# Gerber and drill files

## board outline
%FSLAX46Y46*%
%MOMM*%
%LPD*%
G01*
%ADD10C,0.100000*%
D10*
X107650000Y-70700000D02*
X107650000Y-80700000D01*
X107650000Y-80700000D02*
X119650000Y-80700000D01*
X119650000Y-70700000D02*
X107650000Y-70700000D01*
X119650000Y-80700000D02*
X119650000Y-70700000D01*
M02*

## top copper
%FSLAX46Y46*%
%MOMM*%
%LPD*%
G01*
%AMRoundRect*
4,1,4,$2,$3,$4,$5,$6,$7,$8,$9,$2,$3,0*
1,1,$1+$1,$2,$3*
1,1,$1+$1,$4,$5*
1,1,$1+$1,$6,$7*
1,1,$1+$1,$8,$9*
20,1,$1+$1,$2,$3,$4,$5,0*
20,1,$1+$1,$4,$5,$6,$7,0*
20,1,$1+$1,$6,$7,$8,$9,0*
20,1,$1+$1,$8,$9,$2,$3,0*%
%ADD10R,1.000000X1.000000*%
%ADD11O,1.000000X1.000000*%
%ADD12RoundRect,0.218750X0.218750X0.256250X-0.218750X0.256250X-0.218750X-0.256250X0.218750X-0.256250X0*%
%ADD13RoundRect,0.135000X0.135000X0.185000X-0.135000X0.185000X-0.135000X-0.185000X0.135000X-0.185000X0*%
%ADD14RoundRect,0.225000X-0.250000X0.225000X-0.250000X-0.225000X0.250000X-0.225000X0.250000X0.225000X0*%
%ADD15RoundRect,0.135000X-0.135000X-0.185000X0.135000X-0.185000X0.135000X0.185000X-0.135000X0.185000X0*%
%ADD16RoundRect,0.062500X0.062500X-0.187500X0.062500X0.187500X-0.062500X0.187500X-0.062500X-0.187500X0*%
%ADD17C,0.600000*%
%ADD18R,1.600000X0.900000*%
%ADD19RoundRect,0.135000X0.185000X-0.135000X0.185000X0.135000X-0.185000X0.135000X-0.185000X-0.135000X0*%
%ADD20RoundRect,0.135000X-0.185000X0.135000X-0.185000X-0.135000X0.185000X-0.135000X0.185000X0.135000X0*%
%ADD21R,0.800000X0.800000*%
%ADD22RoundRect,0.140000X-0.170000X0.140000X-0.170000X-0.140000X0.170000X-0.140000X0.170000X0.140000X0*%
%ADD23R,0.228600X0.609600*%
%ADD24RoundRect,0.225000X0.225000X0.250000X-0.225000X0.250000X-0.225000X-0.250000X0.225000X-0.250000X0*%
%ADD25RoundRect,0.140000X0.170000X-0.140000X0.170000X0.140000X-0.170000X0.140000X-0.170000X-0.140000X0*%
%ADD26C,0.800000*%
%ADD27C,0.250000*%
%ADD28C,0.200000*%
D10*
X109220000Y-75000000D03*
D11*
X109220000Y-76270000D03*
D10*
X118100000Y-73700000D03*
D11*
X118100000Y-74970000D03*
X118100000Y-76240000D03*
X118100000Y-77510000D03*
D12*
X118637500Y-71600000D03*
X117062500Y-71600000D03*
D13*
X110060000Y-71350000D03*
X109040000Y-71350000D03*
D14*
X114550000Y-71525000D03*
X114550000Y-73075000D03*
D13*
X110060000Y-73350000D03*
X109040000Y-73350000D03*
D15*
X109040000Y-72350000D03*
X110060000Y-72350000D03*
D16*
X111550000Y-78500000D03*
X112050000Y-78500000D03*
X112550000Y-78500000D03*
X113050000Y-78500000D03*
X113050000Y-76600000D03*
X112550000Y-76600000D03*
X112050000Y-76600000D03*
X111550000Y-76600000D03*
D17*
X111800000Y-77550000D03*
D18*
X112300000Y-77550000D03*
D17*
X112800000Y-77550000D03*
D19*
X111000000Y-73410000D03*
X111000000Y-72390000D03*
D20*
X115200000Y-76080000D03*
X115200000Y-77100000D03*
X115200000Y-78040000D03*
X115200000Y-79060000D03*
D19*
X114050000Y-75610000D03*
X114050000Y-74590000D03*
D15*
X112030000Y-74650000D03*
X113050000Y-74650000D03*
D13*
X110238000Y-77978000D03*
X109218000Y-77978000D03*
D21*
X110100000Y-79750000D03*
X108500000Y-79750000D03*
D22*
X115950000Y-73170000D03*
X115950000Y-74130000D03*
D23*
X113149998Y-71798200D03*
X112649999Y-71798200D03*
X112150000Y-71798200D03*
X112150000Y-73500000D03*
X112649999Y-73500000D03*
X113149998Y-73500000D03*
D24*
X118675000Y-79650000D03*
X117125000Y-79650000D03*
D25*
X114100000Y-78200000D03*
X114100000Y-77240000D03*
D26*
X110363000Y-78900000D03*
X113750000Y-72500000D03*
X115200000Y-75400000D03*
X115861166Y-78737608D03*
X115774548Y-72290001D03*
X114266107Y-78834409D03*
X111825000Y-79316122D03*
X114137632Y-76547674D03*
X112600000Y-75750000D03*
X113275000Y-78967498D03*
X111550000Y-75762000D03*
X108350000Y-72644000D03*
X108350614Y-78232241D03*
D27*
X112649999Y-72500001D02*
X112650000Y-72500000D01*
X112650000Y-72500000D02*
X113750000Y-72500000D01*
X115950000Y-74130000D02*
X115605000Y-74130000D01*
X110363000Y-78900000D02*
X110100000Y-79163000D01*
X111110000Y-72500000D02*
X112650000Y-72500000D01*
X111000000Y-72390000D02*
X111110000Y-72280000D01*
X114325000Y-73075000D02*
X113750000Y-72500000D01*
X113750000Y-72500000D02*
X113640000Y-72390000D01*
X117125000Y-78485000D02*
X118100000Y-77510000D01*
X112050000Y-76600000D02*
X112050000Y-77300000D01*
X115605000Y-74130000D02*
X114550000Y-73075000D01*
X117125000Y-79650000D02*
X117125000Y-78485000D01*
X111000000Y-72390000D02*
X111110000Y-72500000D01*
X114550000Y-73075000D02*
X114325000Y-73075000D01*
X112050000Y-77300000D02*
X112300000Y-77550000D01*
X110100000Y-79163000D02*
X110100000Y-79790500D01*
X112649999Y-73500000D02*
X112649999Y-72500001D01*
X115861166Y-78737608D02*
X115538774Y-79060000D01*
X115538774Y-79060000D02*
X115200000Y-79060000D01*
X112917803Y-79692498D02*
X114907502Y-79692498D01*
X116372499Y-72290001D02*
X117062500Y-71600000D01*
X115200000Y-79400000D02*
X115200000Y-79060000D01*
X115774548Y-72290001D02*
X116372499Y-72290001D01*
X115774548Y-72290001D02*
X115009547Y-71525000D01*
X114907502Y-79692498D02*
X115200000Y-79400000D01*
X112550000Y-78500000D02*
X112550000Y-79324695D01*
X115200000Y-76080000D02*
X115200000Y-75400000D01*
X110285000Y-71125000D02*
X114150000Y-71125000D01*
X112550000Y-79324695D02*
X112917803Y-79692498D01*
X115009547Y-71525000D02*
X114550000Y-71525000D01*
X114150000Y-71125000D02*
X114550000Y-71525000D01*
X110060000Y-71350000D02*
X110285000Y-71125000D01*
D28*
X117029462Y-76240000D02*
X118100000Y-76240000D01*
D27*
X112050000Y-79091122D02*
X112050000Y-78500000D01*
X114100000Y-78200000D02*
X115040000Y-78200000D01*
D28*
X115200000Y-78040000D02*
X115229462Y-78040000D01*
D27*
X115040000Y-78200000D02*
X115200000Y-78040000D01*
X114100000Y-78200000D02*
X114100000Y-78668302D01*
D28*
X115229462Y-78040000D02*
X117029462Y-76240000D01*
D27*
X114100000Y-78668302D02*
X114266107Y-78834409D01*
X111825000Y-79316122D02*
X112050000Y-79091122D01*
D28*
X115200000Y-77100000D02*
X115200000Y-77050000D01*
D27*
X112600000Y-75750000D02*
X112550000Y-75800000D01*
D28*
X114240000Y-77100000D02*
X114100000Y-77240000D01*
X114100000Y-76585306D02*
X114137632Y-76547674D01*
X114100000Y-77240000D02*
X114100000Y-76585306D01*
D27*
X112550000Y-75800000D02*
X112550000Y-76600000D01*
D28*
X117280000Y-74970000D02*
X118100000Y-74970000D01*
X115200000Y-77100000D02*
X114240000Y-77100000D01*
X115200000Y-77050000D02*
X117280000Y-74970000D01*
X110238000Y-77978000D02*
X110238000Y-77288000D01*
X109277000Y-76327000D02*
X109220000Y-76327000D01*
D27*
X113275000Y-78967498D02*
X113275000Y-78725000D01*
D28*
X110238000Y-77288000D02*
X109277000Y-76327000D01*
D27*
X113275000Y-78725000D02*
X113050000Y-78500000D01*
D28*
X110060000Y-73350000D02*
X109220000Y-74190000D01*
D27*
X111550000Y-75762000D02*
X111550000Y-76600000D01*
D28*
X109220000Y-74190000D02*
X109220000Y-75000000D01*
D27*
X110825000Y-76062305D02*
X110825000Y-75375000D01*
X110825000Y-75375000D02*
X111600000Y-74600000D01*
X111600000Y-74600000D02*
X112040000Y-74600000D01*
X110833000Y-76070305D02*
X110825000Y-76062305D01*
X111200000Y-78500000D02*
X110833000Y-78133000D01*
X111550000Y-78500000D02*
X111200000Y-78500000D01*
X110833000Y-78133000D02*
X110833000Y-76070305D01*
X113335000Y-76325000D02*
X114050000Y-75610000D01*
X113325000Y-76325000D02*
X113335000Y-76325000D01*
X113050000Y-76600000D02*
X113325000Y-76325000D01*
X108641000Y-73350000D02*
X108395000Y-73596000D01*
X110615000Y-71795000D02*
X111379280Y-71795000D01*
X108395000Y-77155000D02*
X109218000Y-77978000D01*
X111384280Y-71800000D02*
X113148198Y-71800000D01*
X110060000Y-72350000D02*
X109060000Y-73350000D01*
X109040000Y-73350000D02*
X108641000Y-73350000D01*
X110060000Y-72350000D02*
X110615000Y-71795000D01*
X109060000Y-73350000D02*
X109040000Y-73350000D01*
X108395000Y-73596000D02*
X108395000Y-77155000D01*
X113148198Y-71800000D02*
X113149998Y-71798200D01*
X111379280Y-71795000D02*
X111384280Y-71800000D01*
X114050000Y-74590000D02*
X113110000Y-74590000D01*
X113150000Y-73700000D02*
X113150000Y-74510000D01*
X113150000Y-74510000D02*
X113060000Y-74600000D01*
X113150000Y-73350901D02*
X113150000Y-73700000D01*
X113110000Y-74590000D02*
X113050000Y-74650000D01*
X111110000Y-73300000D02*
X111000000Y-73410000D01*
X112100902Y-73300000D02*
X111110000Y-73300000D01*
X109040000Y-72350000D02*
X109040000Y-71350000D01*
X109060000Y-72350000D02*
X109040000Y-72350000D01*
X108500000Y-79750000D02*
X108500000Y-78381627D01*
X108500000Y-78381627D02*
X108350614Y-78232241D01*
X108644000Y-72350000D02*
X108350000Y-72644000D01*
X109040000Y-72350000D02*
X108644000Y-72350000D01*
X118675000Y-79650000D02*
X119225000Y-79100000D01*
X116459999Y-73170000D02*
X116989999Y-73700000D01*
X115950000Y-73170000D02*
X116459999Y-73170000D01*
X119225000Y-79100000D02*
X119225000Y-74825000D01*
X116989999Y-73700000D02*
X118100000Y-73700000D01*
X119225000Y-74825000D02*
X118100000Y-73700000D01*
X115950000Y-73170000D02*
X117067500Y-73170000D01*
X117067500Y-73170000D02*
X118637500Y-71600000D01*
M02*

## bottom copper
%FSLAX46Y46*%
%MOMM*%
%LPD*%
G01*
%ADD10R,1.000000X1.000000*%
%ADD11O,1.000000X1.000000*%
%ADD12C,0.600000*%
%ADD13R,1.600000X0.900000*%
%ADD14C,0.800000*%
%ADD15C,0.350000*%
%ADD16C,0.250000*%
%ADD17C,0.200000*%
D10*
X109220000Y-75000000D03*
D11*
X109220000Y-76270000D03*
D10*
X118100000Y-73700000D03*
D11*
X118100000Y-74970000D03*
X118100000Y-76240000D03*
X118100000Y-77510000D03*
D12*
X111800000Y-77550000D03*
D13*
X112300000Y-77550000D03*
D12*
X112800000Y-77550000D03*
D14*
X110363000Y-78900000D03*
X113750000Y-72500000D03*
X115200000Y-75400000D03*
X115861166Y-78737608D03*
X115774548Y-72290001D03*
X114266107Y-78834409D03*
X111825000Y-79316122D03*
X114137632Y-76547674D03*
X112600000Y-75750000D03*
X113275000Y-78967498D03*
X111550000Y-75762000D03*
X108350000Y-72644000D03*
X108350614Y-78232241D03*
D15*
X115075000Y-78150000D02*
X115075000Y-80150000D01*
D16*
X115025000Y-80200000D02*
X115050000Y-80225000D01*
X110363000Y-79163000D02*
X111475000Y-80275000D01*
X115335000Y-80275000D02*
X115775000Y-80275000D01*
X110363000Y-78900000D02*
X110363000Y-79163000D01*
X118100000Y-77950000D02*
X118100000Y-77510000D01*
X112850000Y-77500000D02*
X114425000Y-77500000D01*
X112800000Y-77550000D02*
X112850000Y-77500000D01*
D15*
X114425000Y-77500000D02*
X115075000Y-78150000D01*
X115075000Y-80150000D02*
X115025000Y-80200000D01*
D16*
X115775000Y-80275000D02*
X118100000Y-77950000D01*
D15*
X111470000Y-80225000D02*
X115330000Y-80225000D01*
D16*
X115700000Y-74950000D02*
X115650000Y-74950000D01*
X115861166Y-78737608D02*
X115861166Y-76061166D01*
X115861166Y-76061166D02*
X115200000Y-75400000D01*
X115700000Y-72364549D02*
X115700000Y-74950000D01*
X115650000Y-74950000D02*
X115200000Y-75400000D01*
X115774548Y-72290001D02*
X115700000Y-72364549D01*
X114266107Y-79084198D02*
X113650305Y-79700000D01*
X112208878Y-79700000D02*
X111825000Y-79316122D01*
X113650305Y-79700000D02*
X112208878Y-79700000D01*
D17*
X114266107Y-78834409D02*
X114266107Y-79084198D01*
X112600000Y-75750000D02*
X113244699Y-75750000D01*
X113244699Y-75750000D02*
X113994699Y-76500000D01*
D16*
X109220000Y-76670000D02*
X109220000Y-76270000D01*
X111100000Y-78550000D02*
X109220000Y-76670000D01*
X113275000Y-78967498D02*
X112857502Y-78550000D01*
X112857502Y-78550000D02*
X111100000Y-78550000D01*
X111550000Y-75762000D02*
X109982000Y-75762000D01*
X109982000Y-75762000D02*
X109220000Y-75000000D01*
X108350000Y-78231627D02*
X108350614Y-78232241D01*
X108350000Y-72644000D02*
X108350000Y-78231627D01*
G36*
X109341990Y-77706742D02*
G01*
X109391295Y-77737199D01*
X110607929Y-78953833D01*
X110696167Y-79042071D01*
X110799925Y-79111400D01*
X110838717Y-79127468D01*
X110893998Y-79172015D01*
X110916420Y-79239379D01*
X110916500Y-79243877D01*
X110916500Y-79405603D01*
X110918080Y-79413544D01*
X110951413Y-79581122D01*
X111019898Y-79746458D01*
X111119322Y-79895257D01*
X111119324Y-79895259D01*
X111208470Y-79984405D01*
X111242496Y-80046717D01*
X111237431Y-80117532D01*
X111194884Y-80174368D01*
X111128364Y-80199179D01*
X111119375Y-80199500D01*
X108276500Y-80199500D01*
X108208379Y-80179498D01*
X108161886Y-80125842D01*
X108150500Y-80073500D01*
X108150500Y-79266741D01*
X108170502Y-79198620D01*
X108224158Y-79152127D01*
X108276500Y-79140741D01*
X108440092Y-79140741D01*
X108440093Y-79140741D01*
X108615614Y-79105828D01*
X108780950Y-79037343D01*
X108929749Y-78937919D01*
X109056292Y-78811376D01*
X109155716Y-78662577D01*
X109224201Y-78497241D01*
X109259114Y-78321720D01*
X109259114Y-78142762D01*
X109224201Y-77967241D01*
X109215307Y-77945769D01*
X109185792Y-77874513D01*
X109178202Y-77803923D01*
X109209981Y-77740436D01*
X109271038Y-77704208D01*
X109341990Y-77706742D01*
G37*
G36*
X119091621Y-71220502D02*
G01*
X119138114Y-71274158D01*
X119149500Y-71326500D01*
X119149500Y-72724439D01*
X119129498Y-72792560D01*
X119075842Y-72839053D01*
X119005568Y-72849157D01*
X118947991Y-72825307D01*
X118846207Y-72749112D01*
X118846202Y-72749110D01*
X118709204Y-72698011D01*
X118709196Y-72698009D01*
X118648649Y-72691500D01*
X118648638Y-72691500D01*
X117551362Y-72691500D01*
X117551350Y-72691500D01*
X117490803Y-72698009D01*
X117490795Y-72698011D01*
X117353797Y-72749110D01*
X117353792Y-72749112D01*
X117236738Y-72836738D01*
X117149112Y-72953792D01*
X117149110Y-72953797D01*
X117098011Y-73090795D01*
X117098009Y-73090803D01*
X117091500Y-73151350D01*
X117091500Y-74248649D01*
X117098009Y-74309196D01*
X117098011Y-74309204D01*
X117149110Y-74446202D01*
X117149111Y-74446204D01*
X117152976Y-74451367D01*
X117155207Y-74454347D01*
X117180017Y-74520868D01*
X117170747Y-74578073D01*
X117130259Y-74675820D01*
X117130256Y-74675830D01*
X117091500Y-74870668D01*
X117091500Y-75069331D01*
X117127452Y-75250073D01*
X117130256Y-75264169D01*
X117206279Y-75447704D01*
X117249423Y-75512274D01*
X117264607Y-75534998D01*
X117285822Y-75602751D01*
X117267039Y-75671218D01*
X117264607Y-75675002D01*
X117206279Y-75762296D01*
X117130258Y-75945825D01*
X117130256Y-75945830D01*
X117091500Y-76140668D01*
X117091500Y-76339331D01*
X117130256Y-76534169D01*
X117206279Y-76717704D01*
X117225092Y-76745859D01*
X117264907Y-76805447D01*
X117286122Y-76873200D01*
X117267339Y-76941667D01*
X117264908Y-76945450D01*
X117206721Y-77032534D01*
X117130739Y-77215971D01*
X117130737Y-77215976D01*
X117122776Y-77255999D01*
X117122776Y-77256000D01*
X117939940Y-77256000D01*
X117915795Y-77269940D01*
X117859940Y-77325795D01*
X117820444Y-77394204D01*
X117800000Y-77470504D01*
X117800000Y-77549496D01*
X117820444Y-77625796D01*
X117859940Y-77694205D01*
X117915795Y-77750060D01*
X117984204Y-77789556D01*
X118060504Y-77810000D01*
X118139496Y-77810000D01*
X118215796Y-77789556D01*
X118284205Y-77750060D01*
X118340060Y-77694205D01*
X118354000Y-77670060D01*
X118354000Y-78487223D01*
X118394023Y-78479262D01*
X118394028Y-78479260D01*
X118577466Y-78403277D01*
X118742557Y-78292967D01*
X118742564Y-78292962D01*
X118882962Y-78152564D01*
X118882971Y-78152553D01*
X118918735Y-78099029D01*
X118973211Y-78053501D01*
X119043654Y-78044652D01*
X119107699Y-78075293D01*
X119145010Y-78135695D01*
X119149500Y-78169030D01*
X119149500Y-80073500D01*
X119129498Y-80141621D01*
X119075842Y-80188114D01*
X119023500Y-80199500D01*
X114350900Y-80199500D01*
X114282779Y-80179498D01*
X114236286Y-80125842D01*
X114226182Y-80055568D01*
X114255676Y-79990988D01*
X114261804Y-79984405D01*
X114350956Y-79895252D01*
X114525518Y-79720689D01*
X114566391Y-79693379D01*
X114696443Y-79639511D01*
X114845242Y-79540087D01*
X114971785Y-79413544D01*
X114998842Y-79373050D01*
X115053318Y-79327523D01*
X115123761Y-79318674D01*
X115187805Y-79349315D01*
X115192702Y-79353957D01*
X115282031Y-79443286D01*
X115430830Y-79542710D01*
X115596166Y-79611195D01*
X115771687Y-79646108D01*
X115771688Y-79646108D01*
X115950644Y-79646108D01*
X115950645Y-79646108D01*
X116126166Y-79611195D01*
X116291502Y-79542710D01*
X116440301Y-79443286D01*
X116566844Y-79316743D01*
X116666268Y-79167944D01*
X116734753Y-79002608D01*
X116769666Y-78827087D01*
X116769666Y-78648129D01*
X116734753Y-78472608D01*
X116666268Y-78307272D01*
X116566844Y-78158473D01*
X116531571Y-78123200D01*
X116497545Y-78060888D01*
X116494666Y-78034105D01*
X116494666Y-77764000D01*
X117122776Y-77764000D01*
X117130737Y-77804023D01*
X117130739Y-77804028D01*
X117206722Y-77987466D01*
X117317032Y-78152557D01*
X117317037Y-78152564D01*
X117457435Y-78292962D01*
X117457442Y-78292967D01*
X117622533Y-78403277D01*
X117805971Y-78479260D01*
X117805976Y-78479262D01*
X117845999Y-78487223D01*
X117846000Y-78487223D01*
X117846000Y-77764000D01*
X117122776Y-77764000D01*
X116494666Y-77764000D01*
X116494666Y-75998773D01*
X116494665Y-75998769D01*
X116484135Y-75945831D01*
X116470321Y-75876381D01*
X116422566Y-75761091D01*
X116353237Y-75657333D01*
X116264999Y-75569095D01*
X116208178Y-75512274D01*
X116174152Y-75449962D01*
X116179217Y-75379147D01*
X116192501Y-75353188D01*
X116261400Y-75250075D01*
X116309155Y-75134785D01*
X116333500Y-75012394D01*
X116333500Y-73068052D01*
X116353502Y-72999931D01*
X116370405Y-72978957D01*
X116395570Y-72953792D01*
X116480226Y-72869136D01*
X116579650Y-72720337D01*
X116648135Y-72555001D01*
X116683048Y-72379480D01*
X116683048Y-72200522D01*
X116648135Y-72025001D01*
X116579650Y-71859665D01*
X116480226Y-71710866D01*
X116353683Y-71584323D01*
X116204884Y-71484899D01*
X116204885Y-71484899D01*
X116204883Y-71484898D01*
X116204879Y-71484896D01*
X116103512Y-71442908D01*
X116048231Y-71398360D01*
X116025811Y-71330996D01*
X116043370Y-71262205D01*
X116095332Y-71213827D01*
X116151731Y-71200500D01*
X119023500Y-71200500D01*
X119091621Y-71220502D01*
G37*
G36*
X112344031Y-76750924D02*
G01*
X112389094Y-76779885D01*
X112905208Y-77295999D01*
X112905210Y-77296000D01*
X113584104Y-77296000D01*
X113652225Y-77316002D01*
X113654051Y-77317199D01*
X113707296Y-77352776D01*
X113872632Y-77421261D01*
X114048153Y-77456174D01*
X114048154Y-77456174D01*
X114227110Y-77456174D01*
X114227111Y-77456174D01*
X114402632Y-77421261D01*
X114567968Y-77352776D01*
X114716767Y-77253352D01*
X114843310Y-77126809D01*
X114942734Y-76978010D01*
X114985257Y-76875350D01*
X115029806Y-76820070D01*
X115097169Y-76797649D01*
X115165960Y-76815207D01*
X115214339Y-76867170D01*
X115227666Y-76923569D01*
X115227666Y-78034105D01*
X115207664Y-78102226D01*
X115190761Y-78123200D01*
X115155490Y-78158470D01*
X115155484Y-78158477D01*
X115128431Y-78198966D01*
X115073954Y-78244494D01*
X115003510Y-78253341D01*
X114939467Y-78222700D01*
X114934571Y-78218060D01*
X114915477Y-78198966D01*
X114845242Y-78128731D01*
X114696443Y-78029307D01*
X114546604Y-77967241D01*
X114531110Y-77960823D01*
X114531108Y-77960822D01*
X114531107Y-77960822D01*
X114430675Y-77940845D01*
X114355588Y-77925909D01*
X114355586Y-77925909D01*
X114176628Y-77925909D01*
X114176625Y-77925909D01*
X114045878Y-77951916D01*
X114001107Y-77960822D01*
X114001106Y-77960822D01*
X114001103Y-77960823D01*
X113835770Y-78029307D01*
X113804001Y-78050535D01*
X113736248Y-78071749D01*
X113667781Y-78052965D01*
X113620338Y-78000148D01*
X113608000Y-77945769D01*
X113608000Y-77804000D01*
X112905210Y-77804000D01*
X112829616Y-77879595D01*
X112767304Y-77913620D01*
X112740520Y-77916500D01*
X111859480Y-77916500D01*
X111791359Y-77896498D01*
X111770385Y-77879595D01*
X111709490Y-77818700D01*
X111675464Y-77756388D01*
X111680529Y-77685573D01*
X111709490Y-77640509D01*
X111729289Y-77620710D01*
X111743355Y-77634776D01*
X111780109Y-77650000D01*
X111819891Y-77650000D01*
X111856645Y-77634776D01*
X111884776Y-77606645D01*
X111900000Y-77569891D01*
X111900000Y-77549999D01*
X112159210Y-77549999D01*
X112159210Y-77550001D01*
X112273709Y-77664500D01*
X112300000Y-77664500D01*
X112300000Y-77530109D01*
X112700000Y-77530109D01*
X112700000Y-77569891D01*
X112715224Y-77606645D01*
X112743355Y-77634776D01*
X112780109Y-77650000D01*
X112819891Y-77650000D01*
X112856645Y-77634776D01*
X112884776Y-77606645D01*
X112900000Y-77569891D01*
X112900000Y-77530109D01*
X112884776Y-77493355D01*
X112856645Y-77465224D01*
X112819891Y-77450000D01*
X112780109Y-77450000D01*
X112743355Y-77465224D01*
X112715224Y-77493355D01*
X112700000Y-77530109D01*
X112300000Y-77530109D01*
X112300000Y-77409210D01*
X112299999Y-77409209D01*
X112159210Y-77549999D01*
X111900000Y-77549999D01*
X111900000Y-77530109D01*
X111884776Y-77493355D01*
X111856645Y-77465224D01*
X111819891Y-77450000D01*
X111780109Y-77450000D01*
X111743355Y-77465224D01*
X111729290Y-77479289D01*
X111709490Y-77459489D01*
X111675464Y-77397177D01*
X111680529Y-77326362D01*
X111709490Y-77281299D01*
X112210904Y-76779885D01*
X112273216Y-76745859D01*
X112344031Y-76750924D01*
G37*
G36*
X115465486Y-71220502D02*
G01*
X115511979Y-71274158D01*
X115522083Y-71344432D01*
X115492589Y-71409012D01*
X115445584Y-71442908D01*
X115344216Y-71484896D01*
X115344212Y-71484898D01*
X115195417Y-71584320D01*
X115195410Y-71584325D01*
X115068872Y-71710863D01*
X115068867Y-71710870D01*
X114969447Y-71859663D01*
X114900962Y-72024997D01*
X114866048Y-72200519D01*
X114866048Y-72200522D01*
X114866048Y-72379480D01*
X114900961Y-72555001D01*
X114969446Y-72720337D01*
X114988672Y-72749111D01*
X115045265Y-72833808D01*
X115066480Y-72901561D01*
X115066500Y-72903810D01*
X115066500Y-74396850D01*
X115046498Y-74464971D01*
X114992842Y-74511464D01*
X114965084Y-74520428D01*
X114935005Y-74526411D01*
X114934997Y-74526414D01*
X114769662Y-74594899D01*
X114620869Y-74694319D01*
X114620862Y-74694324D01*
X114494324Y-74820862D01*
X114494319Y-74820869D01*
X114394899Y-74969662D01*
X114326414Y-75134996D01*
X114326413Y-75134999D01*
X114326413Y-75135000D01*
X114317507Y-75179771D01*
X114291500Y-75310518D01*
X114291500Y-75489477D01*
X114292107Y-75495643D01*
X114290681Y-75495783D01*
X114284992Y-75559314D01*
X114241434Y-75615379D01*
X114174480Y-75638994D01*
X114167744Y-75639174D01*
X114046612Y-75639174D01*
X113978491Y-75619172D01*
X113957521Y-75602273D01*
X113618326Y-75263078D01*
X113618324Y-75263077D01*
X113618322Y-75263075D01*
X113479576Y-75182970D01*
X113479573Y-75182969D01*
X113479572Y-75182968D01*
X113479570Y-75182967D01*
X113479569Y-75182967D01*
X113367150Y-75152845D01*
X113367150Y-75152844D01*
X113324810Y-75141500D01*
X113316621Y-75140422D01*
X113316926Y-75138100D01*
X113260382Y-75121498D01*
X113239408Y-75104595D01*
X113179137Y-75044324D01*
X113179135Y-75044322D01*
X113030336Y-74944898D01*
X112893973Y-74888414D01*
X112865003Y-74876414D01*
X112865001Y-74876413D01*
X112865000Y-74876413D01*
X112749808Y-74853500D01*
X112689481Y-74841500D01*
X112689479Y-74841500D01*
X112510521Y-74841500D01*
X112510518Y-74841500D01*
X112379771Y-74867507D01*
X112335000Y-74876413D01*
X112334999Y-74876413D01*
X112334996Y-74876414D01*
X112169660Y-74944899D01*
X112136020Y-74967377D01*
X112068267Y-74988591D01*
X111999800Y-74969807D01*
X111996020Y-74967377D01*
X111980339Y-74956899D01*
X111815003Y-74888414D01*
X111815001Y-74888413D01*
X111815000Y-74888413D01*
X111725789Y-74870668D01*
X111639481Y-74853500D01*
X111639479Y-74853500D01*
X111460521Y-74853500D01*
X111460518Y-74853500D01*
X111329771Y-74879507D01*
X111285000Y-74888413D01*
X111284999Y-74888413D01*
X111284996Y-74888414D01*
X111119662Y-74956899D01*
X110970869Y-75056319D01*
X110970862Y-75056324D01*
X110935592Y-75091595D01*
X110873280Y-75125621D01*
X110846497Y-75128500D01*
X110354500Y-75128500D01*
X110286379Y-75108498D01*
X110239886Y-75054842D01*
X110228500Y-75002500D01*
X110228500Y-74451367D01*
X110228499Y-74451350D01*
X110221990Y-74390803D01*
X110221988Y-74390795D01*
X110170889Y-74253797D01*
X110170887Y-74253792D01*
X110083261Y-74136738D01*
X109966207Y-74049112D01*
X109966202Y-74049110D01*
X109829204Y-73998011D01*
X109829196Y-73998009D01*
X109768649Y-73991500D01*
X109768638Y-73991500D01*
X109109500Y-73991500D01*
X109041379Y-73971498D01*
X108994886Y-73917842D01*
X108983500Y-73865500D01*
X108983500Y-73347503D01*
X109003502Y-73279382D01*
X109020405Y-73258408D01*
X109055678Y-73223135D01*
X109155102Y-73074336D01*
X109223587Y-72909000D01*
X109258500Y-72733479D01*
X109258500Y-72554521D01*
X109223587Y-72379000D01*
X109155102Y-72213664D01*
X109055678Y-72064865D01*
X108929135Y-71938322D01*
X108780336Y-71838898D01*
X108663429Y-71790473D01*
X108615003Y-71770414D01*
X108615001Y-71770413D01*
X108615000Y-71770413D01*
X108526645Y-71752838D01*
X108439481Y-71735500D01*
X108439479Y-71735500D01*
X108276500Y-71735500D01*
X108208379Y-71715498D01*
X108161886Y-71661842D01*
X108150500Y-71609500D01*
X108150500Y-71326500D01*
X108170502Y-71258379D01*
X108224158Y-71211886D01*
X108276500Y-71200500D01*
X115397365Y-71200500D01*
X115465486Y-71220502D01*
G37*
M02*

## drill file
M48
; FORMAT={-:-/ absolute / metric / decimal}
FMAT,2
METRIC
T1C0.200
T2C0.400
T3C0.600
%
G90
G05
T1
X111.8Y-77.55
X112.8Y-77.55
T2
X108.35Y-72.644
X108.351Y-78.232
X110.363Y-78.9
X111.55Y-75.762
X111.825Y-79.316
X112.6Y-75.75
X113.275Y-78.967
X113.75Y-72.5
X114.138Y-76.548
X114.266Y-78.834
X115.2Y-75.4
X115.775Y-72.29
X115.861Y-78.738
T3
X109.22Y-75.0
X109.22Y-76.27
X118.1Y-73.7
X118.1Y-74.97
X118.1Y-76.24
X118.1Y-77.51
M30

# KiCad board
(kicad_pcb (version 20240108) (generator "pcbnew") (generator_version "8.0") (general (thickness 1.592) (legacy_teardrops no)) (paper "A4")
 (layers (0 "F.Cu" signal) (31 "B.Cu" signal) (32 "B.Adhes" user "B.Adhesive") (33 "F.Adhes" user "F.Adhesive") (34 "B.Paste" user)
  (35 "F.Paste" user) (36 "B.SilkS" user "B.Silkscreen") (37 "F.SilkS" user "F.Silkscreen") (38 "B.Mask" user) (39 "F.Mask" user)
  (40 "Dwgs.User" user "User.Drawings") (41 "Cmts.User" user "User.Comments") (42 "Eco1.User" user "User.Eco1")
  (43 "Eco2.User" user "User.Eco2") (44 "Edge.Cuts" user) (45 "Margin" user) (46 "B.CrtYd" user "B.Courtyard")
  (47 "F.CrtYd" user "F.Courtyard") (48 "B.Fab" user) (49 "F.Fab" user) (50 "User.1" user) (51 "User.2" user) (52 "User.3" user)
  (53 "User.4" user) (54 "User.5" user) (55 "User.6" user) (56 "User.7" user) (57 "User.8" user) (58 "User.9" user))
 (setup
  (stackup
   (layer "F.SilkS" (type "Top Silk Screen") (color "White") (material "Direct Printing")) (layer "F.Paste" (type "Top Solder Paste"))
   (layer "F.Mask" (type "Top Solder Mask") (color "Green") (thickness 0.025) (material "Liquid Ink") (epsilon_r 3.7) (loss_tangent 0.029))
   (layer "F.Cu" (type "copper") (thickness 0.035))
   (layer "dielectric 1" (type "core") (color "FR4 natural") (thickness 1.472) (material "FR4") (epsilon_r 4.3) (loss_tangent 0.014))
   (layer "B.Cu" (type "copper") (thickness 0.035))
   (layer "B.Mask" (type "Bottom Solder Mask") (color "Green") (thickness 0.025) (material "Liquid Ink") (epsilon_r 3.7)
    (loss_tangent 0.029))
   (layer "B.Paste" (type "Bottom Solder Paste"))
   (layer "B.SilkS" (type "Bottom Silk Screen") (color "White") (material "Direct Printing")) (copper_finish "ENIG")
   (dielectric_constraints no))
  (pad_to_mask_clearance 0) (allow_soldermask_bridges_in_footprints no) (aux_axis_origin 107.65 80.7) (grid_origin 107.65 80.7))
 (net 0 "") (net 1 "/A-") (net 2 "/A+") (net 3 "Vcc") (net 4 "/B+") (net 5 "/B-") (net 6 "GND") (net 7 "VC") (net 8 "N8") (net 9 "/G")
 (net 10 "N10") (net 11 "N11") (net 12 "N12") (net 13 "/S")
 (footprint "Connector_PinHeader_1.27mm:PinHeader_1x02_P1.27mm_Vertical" (layer "F.Cu") (at 109.22 75)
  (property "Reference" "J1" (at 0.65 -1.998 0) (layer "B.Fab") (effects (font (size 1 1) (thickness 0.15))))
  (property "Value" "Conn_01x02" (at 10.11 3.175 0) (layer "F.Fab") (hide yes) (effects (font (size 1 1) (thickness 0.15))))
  (pad "1" thru_hole rect (at 0 0) (size 1 1) (drill 0.6) (layers "*.Cu" "*.Mask") (remove_unused_layers no) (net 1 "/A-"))
  (pad "2" thru_hole oval (at 0 1.27) (size 1 1) (drill 0.6) (layers "*.Cu" "*.Mask") (remove_unused_layers no) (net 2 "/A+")))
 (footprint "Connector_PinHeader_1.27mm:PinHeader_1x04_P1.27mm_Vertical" (layer "F.Cu") (at 118.1 73.7)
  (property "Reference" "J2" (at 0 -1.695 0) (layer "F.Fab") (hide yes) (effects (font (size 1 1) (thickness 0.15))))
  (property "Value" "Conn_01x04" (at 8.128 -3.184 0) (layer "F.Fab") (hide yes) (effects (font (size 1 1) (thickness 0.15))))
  (pad "1" thru_hole rect (at 0 0) (size 1 1) (drill 0.6) (layers "*.Cu" "*.Mask") (remove_unused_layers no) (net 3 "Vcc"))
  (pad "2" thru_hole oval (at 0 1.27) (size 1 1) (drill 0.6) (layers "*.Cu" "*.Mask") (remove_unused_layers no) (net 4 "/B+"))
  (pad "3" thru_hole oval (at 0 2.54) (size 1 1) (drill 0.6) (layers "*.Cu" "*.Mask") (remove_unused_layers no) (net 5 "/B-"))
  (pad "4" thru_hole oval (at 0 3.81) (size 1 1) (drill 0.6) (layers "*.Cu" "*.Mask") (remove_unused_layers no) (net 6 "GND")))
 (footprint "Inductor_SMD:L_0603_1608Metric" (layer "F.Cu") (at 117.85 71.6 180)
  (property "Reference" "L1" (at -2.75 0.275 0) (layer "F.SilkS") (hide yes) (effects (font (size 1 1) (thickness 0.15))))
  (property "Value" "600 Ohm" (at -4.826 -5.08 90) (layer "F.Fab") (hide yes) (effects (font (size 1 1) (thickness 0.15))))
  (pad "1" smd roundrect (at -0.7875 0 180) (size 0.875 0.95) (layers "F.Cu" "F.Paste" "F.Mask") (roundrect_rratio 0.25) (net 3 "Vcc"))
  (pad "2" smd roundrect (at 0.7875 0 180) (size 0.875 0.95) (layers "F.Cu" "F.Paste" "F.Mask") (roundrect_rratio 0.25) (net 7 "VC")))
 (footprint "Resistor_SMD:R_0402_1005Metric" (layer "F.Cu") (at 109.55 71.35 180)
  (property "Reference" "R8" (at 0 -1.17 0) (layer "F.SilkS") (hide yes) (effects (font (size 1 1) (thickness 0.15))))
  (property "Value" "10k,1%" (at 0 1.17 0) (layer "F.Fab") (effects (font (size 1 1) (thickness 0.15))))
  (pad "1" smd roundrect (at -0.51 0 180) (size 0.54 0.64) (layers "F.Cu" "F.Paste" "F.Mask") (roundrect_rratio 0.25) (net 7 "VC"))
  (pad "2" smd roundrect (at 0.51 0 180) (size 0.54 0.64) (layers "F.Cu" "F.Paste" "F.Mask") (roundrect_rratio 0.25) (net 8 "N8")))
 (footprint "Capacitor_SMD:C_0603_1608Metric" (layer "F.Cu") (at 114.55 72.3 -90)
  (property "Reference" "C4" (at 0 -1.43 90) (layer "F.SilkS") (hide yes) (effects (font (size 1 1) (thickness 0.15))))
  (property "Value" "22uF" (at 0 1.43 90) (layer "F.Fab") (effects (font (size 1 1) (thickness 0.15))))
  (pad "1" smd roundrect (at -0.775 0 270) (size 0.9 0.95) (layers "F.Cu" "F.Paste" "F.Mask") (roundrect_rratio 0.25) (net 7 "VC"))
  (pad "2" smd roundrect (at 0.775 0 270) (size 0.9 0.95) (layers "F.Cu" "F.Paste" "F.Mask") (roundrect_rratio 0.25) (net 6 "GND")))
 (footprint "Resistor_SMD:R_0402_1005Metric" (layer "F.Cu") (at 109.55 73.35 180)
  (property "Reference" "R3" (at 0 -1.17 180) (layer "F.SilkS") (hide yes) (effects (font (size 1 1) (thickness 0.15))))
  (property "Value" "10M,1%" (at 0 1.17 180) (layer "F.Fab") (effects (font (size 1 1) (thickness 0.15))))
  (pad "1" smd roundrect (at -0.51 0 180) (size 0.54 0.64) (layers "F.Cu" "F.Paste" "F.Mask") (roundrect_rratio 0.25) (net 1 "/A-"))
  (pad "2" smd roundrect (at 0.51 0 180) (size 0.54 0.64) (layers "F.Cu" "F.Paste" "F.Mask") (roundrect_rratio 0.25) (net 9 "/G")))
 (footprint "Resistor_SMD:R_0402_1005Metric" (layer "F.Cu") (at 109.55 72.35)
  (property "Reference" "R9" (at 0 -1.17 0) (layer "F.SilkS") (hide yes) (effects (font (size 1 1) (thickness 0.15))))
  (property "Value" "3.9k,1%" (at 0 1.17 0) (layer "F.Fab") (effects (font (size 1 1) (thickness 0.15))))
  (pad "1" smd roundrect (at -0.51 0) (size 0.54 0.64) (layers "F.Cu" "F.Paste" "F.Mask") (roundrect_rratio 0.25) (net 8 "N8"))
  (pad "2" smd roundrect (at 0.51 0) (size 0.54 0.64) (layers "F.Cu" "F.Paste" "F.Mask") (roundrect_rratio 0.25) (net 9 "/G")))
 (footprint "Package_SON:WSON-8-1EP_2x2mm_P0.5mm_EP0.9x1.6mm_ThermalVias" (layer "F.Cu") (at 112.3 77.55 90)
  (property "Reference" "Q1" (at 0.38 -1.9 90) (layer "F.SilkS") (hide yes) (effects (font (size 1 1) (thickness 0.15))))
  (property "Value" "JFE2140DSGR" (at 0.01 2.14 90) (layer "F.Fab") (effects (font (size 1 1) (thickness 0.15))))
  (pad "" smd rect (at 0 -0.4 90) (size 0.75 0.65) (layers "F.Paste"))
  (pad "" smd rect (at 0 0.4 90) (size 0.75 0.65) (layers "F.Paste"))
  (pad "1" smd roundrect (at -0.95 -0.75 90) (size 0.5 0.25) (layers "F.Cu" "F.Paste" "F.Mask") (roundrect_rratio 0.25) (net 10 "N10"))
  (pad "2" smd roundrect (at -0.95 -0.25 90) (size 0.5 0.25) (layers "F.Cu" "F.Paste" "F.Mask") (roundrect_rratio 0.25) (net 5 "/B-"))
  (pad "3" smd roundrect (at -0.95 0.25 90) (size 0.5 0.25) (layers "F.Cu" "F.Paste" "F.Mask") (roundrect_rratio 0.25) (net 7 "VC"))
  (pad "4" smd roundrect (at -0.95 0.75 90) (size 0.5 0.25) (layers "F.Cu" "F.Paste" "F.Mask") (roundrect_rratio 0.25) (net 2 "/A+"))
  (pad "5" smd roundrect (at 0.95 0.75 90) (size 0.5 0.25) (layers "F.Cu" "F.Paste" "F.Mask") (roundrect_rratio 0.25) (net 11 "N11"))
  (pad "6" smd roundrect (at 0.95 0.25 90) (size 0.5 0.25) (layers "F.Cu" "F.Paste" "F.Mask") (roundrect_rratio 0.25) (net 4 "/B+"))
  (pad "7" smd roundrect (at 0.95 -0.25 90) (size 0.5 0.25) (layers "F.Cu" "F.Paste" "F.Mask") (roundrect_rratio 0.25) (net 6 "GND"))
  (pad "8" smd roundrect (at 0.95 -0.75 90) (size 0.5 0.25) (layers "F.Cu" "F.Paste" "F.Mask") (roundrect_rratio 0.25) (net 1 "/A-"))
  (pad "9" thru_hole circle (at 0 -0.5 90) (size 0.6 0.6) (drill 0.2) (layers "*.Cu") (remove_unused_layers no) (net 6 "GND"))
  (pad "9" smd rect (at 0 0 90) (size 0.9 1.6) (layers "F.Cu" "F.Mask") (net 6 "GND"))
  (pad "9" smd rect (at 0 0 90) (size 0.9 1.6) (layers "B.Cu") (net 6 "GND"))
  (pad "9" thru_hole circle (at 0 0.5 90) (size 0.6 0.6) (drill 0.2) (layers "*.Cu") (remove_unused_layers no) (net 6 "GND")))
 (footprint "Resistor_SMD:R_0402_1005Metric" (layer "F.Cu") (at 111 72.9 90)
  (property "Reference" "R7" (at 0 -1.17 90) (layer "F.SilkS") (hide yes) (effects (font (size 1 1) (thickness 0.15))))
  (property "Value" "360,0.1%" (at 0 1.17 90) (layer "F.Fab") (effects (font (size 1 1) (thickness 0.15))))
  (pad "1" smd roundrect (at -0.51 0 90) (size 0.54 0.64) (layers "F.Cu" "F.Paste" "F.Mask") (roundrect_rratio 0.25) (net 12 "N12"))
  (pad "2" smd roundrect (at 0.51 0 90) (size 0.54 0.64) (layers "F.Cu" "F.Paste" "F.Mask") (roundrect_rratio 0.25) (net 6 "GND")))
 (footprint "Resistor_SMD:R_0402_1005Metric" (layer "F.Cu") (at 115.2 76.59 -90)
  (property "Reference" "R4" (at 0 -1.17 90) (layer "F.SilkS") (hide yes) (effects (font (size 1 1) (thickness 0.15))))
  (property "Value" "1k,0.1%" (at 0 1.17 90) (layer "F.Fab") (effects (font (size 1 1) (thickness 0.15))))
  (pad "1" smd roundrect (at -0.51 0 270) (size 0.54 0.64) (layers "F.Cu" "F.Paste" "F.Mask") (roundrect_rratio 0.25) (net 7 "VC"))
  (pad "2" smd roundrect (at 0.51 0 270) (size 0.54 0.64) (layers "F.Cu" "F.Paste" "F.Mask") (roundrect_rratio 0.25) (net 4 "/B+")))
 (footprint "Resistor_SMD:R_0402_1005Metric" (layer "F.Cu") (at 115.2 78.55 -90)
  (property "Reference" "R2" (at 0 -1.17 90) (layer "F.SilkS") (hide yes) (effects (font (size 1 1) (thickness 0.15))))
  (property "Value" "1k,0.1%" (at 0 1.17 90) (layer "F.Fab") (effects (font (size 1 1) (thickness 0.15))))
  (pad "1" smd roundrect (at -0.51 0 270) (size 0.54 0.64) (layers "F.Cu" "F.Paste" "F.Mask") (roundrect_rratio 0.25) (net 5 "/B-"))
  (pad "2" smd roundrect (at 0.51 0 270) (size 0.54 0.64) (layers "F.Cu" "F.Paste" "F.Mask") (roundrect_rratio 0.25) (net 7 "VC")))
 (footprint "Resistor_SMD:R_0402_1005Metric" (layer "F.Cu") (at 114.05 75.1 90)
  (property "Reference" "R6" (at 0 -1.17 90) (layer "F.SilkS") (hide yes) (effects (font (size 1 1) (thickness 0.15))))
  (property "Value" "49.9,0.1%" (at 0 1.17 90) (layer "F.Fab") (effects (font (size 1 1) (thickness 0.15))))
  (pad "1" smd roundrect (at -0.51 0 90) (size 0.54 0.64) (layers "F.Cu" "F.Paste" "F.Mask") (roundrect_rratio 0.25) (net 11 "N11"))
  (pad "2" smd roundrect (at 0.51 0 90) (size 0.54 0.64) (layers "F.Cu" "F.Paste" "F.Mask") (roundrect_rratio 0.25) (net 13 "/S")))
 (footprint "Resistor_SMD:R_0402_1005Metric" (layer "F.Cu") (at 112.54 74.65)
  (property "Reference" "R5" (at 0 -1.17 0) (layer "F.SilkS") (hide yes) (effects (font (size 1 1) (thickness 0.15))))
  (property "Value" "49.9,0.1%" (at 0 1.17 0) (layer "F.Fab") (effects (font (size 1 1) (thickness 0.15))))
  (pad "1" smd roundrect (at -0.51 0) (size 0.54 0.64) (layers "F.Cu" "F.Paste" "F.Mask") (roundrect_rratio 0.25) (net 10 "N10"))
  (pad "2" smd roundrect (at 0.51 0) (size 0.54 0.64) (layers "F.Cu" "F.Paste" "F.Mask") (roundrect_rratio 0.25) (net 13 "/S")))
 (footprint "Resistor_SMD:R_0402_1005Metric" (layer "F.Cu") (at 109.728 77.978 180)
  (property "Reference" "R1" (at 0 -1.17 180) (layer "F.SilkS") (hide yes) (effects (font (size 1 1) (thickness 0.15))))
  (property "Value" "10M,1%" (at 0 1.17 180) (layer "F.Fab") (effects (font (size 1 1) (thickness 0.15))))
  (pad "1" smd roundrect (at -0.51 0 180) (size 0.54 0.64) (layers "F.Cu" "F.Paste" "F.Mask") (roundrect_rratio 0.25) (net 2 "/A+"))
  (pad "2" smd roundrect (at 0.51 0 180) (size 0.54 0.64) (layers "F.Cu" "F.Paste" "F.Mask") (roundrect_rratio 0.25) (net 9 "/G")))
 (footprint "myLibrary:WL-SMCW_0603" (layer "F.Cu") (at 109.3 79.75 180)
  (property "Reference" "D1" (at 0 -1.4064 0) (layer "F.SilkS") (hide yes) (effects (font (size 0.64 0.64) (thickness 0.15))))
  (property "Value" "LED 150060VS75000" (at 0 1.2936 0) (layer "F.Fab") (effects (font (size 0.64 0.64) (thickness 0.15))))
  (pad "1" smd rect (at -0.8 0 180) (size 0.8 0.8) (layers "F.Cu" "F.Paste" "F.Mask") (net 6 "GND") (solder_mask_margin 0.102))
  (pad "2" smd rect (at 0.8 0 180) (size 0.8 0.8) (layers "F.Cu" "F.Paste" "F.Mask") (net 8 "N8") (solder_mask_margin 0.102)))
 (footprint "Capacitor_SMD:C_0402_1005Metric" (layer "F.Cu") (at 115.95 73.65 -90)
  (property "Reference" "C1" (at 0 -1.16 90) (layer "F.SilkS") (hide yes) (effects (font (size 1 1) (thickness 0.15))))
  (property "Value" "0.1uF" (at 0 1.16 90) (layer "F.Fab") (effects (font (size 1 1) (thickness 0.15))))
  (pad "1" smd roundrect (at -0.48 0 270) (size 0.56 0.62) (layers "F.Cu" "F.Paste" "F.Mask") (roundrect_rratio 0.25) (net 3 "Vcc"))
  (pad "2" smd roundrect (at 0.48 0 270) (size 0.56 0.62) (layers "F.Cu" "F.Paste" "F.Mask") (roundrect_rratio 0.25) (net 6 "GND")))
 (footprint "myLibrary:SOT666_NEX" (layer "F.Cu") (at 112.649999 72.6491 -90)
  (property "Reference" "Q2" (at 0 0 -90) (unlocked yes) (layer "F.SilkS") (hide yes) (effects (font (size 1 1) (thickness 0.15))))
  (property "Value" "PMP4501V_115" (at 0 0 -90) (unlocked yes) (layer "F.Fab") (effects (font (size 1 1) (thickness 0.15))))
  (pad "1" smd rect (at -0.8509 -0.499999 270) (size 0.6096 0.2286) (layers "F.Cu" "F.Paste" "F.Mask") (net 9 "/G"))
  (pad "2" smd rect (at -0.8509 0 270) (size 0.6096 0.2286) (layers "F.Cu" "F.Paste" "F.Mask") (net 9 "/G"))
  (pad "3" smd rect (at -0.8509 0.499999 270) (size 0.6096 0.2286) (layers "F.Cu" "F.Paste" "F.Mask") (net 9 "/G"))
  (pad "4" smd rect (at 0.8509 0.499999 270) (size 0.6096 0.2286) (layers "F.Cu" "F.Paste" "F.Mask") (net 12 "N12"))
  (pad "5" smd rect (at 0.8509 0 270) (size 0.6096 0.2286) (layers "F.Cu" "F.Paste" "F.Mask") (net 6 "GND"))
  (pad "6" smd rect (at 0.8509 -0.499999 270) (size 0.6096 0.2286) (layers "F.Cu" "F.Paste" "F.Mask") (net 13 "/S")))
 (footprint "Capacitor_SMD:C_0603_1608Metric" (layer "F.Cu") (at 117.9 79.65 180)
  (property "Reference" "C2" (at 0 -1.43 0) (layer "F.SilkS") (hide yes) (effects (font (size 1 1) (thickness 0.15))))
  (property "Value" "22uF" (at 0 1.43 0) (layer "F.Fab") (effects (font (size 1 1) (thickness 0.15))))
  (pad "1" smd roundrect (at -0.775 0 180) (size 0.9 0.95) (layers "F.Cu" "F.Paste" "F.Mask") (roundrect_rratio 0.25) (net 3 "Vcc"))
  (pad "2" smd roundrect (at 0.775 0 180) (size 0.9 0.95) (layers "F.Cu" "F.Paste" "F.Mask") (roundrect_rratio 0.25) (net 6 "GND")))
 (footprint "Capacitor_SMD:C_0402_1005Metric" (layer "F.Cu") (at 114.1 77.72 90)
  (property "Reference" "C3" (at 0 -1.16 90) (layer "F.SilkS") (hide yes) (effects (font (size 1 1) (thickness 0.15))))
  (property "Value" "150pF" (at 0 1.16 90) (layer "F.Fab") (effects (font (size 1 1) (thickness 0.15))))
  (pad "1" smd roundrect (at -0.48 0 90) (size 0.56 0.62) (layers "F.Cu" "F.Paste" "F.Mask") (roundrect_rratio 0.25) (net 5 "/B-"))
  (pad "2" smd roundrect (at 0.48 0 90) (size 0.56 0.62) (layers "F.Cu" "F.Paste" "F.Mask") (roundrect_rratio 0.25) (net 4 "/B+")))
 (gr_line (start 107.65 70.7) (end 107.65 80.7) (stroke (width 0.1) (type solid)) (layer "Edge.Cuts"))
 (gr_line (start 107.65 80.7) (end 119.65 80.7) (stroke (width 0.1) (type solid)) (layer "Edge.Cuts"))
 (gr_line (start 119.65 70.7) (end 107.65 70.7) (stroke (width 0.1) (type solid)) (layer "Edge.Cuts"))
 (gr_line (start 119.65 80.7) (end 119.65 70.7) (stroke (width 0.1) (type solid)) (layer "Edge.Cuts"))
 (segment (start 112.649999 72.500001) (end 112.65 72.5) (width 0.25) (layer "F.Cu") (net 6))
 (segment (start 112.65 72.5) (end 113.75 72.5) (width 0.25) (layer "F.Cu") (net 6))
 (segment (start 115.95 74.13) (end 115.605 74.13) (width 0.25) (layer "F.Cu") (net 6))
 (segment (start 110.363 78.9) (end 110.1 79.163) (width 0.25) (layer "F.Cu") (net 6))
 (segment (start 111.11 72.5) (end 112.65 72.5) (width 0.25) (layer "F.Cu") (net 6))
 (segment (start 111 72.39) (end 111.11 72.28) (width 0.25) (layer "F.Cu") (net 6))
 (segment (start 114.325 73.075) (end 113.75 72.5) (width 0.25) (layer "F.Cu") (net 6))
 (segment (start 113.75 72.5) (end 113.64 72.39) (width 0.25) (layer "F.Cu") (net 6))
 (segment (start 117.125 78.485) (end 118.1 77.51) (width 0.25) (layer "F.Cu") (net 6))
 (segment (start 112.05 76.6) (end 112.05 77.3) (width 0.25) (layer "F.Cu") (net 6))
 (segment (start 115.605 74.13) (end 114.55 73.075) (width 0.25) (layer "F.Cu") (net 6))
 (segment (start 117.125 79.65) (end 117.125 78.485) (width 0.25) (layer "F.Cu") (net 6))
 (segment (start 111 72.39) (end 111.11 72.5) (width 0.25) (layer "F.Cu") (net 6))
 (segment (start 114.55 73.075) (end 114.325 73.075) (width 0.25) (layer "F.Cu") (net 6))
 (segment (start 112.05 77.3) (end 112.3 77.55) (width 0.25) (layer "F.Cu") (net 6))
 (segment (start 110.1 79.163) (end 110.1 79.7905) (width 0.25) (layer "F.Cu") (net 6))
 (segment (start 112.649999 73.5) (end 112.649999 72.500001) (width 0.25) (layer "F.Cu") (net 6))
 (via (at 110.363 78.9) (size 0.8) (drill 0.4) (layers "F.Cu" "B.Cu") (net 6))
 (via (at 113.75 72.5) (size 0.8) (drill 0.4) (layers "F.Cu" "B.Cu") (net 6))
 (segment (start 115.075 78.15) (end 115.075 80.15) (width 0.35) (layer "B.Cu") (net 6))
 (segment (start 115.025 80.2) (end 115.05 80.225) (width 0.25) (layer "B.Cu") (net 6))
 (segment (start 110.363 79.163) (end 111.475 80.275) (width 0.25) (layer "B.Cu") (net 6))
 (segment (start 115.335 80.275) (end 115.775 80.275) (width 0.25) (layer "B.Cu") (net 6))
 (segment (start 110.363 78.9) (end 110.363 79.163) (width 0.25) (layer "B.Cu") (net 6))
 (segment (start 118.1 77.95) (end 118.1 77.51) (width 0.25) (layer "B.Cu") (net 6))
 (segment (start 112.85 77.5) (end 114.425 77.5) (width 0.25) (layer "B.Cu") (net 6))
 (segment (start 112.8 77.55) (end 112.85 77.5) (width 0.25) (layer "B.Cu") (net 6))
 (segment (start 114.425 77.5) (end 115.075 78.15) (width 0.35) (layer "B.Cu") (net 6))
 (segment (start 115.075 80.15) (end 115.025 80.2) (width 0.35) (layer "B.Cu") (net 6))
 (segment (start 115.775 80.275) (end 118.1 77.95) (width 0.25) (layer "B.Cu") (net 6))
 (segment (start 111.47 80.225) (end 115.33 80.225) (width 0.35) (layer "B.Cu") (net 6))
 (segment (start 115.861166 78.737608) (end 115.538774 79.06) (width 0.25) (layer "F.Cu") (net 7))
 (segment (start 115.538774 79.06) (end 115.2 79.06) (width 0.25) (layer "F.Cu") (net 7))
 (segment (start 112.917803 79.692498) (end 114.907502 79.692498) (width 0.25) (layer "F.Cu") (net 7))
 (segment (start 116.372499 72.290001) (end 117.0625 71.6) (width 0.25) (layer "F.Cu") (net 7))
 (segment (start 115.2 79.4) (end 115.2 79.06) (width 0.25) (layer "F.Cu") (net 7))
 (segment (start 115.774548 72.290001) (end 116.372499 72.290001) (width 0.25) (layer "F.Cu") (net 7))
 (segment (start 115.774548 72.290001) (end 115.009547 71.525) (width 0.25) (layer "F.Cu") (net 7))
 (segment (start 114.907502 79.692498) (end 115.2 79.4) (width 0.25) (layer "F.Cu") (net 7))
 (segment (start 112.55 78.5) (end 112.55 79.324695) (width 0.25) (layer "F.Cu") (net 7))
 (segment (start 115.2 76.08) (end 115.2 75.4) (width 0.25) (layer "F.Cu") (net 7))
 (segment (start 110.285 71.125) (end 114.15 71.125) (width 0.25) (layer "F.Cu") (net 7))
 (segment (start 112.55 79.324695) (end 112.917803 79.692498) (width 0.25) (layer "F.Cu") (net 7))
 (segment (start 115.009547 71.525) (end 114.55 71.525) (width 0.25) (layer "F.Cu") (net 7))
 (segment (start 114.15 71.125) (end 114.55 71.525) (width 0.25) (layer "F.Cu") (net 7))
 (segment (start 110.06 71.35) (end 110.285 71.125) (width 0.25) (layer "F.Cu") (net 7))
 (via (at 115.2 75.4) (size 0.8) (drill 0.4) (layers "F.Cu" "B.Cu") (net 7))
 (via (at 115.861166 78.737608) (size 0.8) (drill 0.4) (layers "F.Cu" "B.Cu") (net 7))
 (via (at 115.774548 72.290001) (size 0.8) (drill 0.4) (layers "F.Cu" "B.Cu") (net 7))
 (segment (start 115.7 74.95) (end 115.65 74.95) (width 0.25) (layer "B.Cu") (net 7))
 (segment (start 115.861166 78.737608) (end 115.861166 76.061166) (width 0.25) (layer "B.Cu") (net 7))
 (segment (start 115.861166 76.061166) (end 115.2 75.4) (width 0.25) (layer "B.Cu") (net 7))
 (segment (start 115.7 72.364549) (end 115.7 74.95) (width 0.25) (layer "B.Cu") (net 7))
 (segment (start 115.65 74.95) (end 115.2 75.4) (width 0.25) (layer "B.Cu") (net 7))
 (segment (start 115.774548 72.290001) (end 115.7 72.364549) (width 0.25) (layer "B.Cu") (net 7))
 (segment (start 117.029462 76.24) (end 118.1 76.24) (width 0.2) (layer "F.Cu") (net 5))
 (segment (start 112.05 79.091122) (end 112.05 78.5) (width 0.25) (layer "F.Cu") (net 5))
 (segment (start 114.1 78.2) (end 115.04 78.2) (width 0.25) (layer "F.Cu") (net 5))
 (segment (start 115.2 78.04) (end 115.229462 78.04) (width 0.2) (layer "F.Cu") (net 5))
 (segment (start 115.04 78.2) (end 115.2 78.04) (width 0.25) (layer "F.Cu") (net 5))
 (segment (start 114.1 78.2) (end 114.1 78.668302) (width 0.25) (layer "F.Cu") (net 5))
 (segment (start 115.229462 78.04) (end 117.029462 76.24) (width 0.2) (layer "F.Cu") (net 5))
 (segment (start 114.1 78.668302) (end 114.266107 78.834409) (width 0.25) (layer "F.Cu") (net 5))
 (segment (start 111.825 79.316122) (end 112.05 79.091122) (width 0.25) (layer "F.Cu") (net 5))
 (via (at 114.266107 78.834409) (size 0.8) (drill 0.4) (layers "F.Cu" "B.Cu") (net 5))
 (via (at 111.825 79.316122) (size 0.8) (drill 0.4) (layers "F.Cu" "B.Cu") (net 5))
 (segment (start 114.266107 79.084198) (end 113.650305 79.7) (width 0.25) (layer "B.Cu") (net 5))
 (segment (start 112.208878 79.7) (end 111.825 79.316122) (width 0.25) (layer "B.Cu") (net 5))
 (segment (start 113.650305 79.7) (end 112.208878 79.7) (width 0.25) (layer "B.Cu") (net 5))
 (segment (start 114.266107 78.834409) (end 114.266107 79.084198) (width 0.2) (layer "B.Cu") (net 5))
 (segment (start 115.2 77.1) (end 115.2 77.05) (width 0.2) (layer "F.Cu") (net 4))
 (segment (start 112.6 75.75) (end 112.55 75.8) (width 0.25) (layer "F.Cu") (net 4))
 (segment (start 114.24 77.1) (end 114.1 77.24) (width 0.2) (layer "F.Cu") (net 4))
 (segment (start 114.1 76.585306) (end 114.137632 76.547674) (width 0.2) (layer "F.Cu") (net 4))
 (segment (start 114.1 77.24) (end 114.1 76.585306) (width 0.2) (layer "F.Cu") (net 4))
 (segment (start 112.55 75.8) (end 112.55 76.6) (width 0.25) (layer "F.Cu") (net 4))
 (segment (start 117.28 74.97) (end 118.1 74.97) (width 0.2) (layer "F.Cu") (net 4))
 (segment (start 115.2 77.1) (end 114.24 77.1) (width 0.2) (layer "F.Cu") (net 4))
 (segment (start 115.2 77.05) (end 117.28 74.97) (width 0.2) (layer "F.Cu") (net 4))
 (via (at 114.137632 76.547674) (size 0.8) (drill 0.4) (layers "F.Cu" "B.Cu") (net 4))
 (via (at 112.6 75.75) (size 0.8) (drill 0.4) (layers "F.Cu" "B.Cu") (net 4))
 (segment (start 112.6 75.75) (end 113.244699 75.75) (width 0.2) (layer "B.Cu") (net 4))
 (segment (start 113.244699 75.75) (end 113.994699 76.5) (width 0.2) (layer "B.Cu") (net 4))
 (segment (start 110.238 77.978) (end 110.238 77.288) (width 0.2) (layer "F.Cu") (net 2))
 (segment (start 109.277 76.327) (end 109.22 76.327) (width 0.2) (layer "F.Cu") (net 2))
 (segment (start 113.275 78.967498) (end 113.275 78.725) (width 0.25) (layer "F.Cu") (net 2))
 (segment (start 110.238 77.288) (end 109.277 76.327) (width 0.2) (layer "F.Cu") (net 2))
 (segment (start 113.275 78.725) (end 113.05 78.5) (width 0.25) (layer "F.Cu") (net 2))
 (via (at 113.275 78.967498) (size 0.8) (drill 0.4) (layers "F.Cu" "B.Cu") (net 2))
 (segment (start 109.22 76.67) (end 109.22 76.27) (width 0.25) (layer "B.Cu") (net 2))
 (segment (start 111.1 78.55) (end 109.22 76.67) (width 0.25) (layer "B.Cu") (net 2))
 (segment (start 113.275 78.967498) (end 112.857502 78.55) (width 0.25) (layer "B.Cu") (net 2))
 (segment (start 112.857502 78.55) (end 111.1 78.55) (width 0.25) (layer "B.Cu") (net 2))
 (segment (start 110.06 73.35) (end 109.22 74.19) (width 0.2) (layer "F.Cu") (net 1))
 (segment (start 111.55 75.762) (end 111.55 76.6) (width 0.25) (layer "F.Cu") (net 1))
 (segment (start 109.22 74.19) (end 109.22 75) (width 0.2) (layer "F.Cu") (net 1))
 (via (at 111.55 75.762) (size 0.8) (drill 0.4) (layers "F.Cu" "B.Cu") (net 1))
 (segment (start 111.55 75.762) (end 109.982 75.762) (width 0.25) (layer "B.Cu") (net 1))
 (segment (start 109.982 75.762) (end 109.22 75) (width 0.25) (layer "B.Cu") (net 1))
 (segment (start 110.825 76.062305) (end 110.825 75.375) (width 0.25) (layer "F.Cu") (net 10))
 (segment (start 110.825 75.375) (end 111.6 74.6) (width 0.25) (layer "F.Cu") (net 10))
 (segment (start 111.6 74.6) (end 112.04 74.6) (width 0.25) (layer "F.Cu") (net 10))
 (segment (start 110.833 76.070305) (end 110.825 76.062305) (width 0.25) (layer "F.Cu") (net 10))
 (segment (start 111.2 78.5) (end 110.833 78.133) (width 0.25) (layer "F.Cu") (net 10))
 (segment (start 111.55 78.5) (end 111.2 78.5) (width 0.25) (layer "F.Cu") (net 10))
 (segment (start 110.833 78.133) (end 110.833 76.070305) (width 0.25) (layer "F.Cu") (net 10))
 (segment (start 113.335 76.325) (end 114.05 75.61) (width 0.25) (layer "F.Cu") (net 11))
 (segment (start 113.325 76.325) (end 113.335 76.325) (width 0.25) (layer "F.Cu") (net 11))
 (segment (start 113.05 76.6) (end 113.325 76.325) (width 0.25) (layer "F.Cu") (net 11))
 (segment (start 108.641 73.35) (end 108.395 73.596) (width 0.25) (layer "F.Cu") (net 9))
 (segment (start 110.615 71.795) (end 111.37928 71.795) (width 0.25) (layer "F.Cu") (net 9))
 (segment (start 108.395 77.155) (end 109.218 77.978) (width 0.25) (layer "F.Cu") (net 9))
 (segment (start 111.38428 71.8) (end 113.148198 71.8) (width 0.25) (layer "F.Cu") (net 9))
 (segment (start 110.06 72.35) (end 109.06 73.35) (width 0.25) (layer "F.Cu") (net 9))
 (segment (start 109.04 73.35) (end 108.641 73.35) (width 0.25) (layer "F.Cu") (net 9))
 (segment (start 110.06 72.35) (end 110.615 71.795) (width 0.25) (layer "F.Cu") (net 9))
 (segment (start 109.06 73.35) (end 109.04 73.35) (width 0.25) (layer "F.Cu") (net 9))
 (segment (start 108.395 73.596) (end 108.395 77.155) (width 0.25) (layer "F.Cu") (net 9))
 (segment (start 113.148198 71.8) (end 113.149998 71.7982) (width 0.25) (layer "F.Cu") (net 9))
 (segment (start 111.37928 71.795) (end 111.38428 71.8) (width 0.25) (layer "F.Cu") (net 9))
 (segment (start 114.05 74.59) (end 113.11 74.59) (width 0.25) (layer "F.Cu") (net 13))
 (segment (start 113.15 73.7) (end 113.15 74.51) (width 0.25) (layer "F.Cu") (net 13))
 (segment (start 113.15 74.51) (end 113.06 74.6) (width 0.25) (layer "F.Cu") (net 13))
 (segment (start 113.15 73.350901) (end 113.15 73.7) (width 0.25) (layer "F.Cu") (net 13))
 (segment (start 113.11 74.59) (end 113.05 74.65) (width 0.25) (layer "F.Cu") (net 13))
 (segment (start 111.11 73.3) (end 111 73.41) (width 0.25) (layer "F.Cu") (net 12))
 (segment (start 112.100902 73.3) (end 111.11 73.3) (width 0.25) (layer "F.Cu") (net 12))
 (segment (start 109.04 72.35) (end 109.04 71.35) (width 0.25) (layer "F.Cu") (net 8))
 (segment (start 109.06 72.35) (end 109.04 72.35) (width 0.25) (layer "F.Cu") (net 8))
 (segment (start 108.5 79.75) (end 108.5 78.381627) (width 0.25) (layer "F.Cu") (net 8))
 (segment (start 108.5 78.381627) (end 108.350614 78.232241) (width 0.25) (layer "F.Cu") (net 8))
 (segment (start 108.644 72.35) (end 108.35 72.644) (width 0.25) (layer "F.Cu") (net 8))
 (segment (start 109.04 72.35) (end 108.644 72.35) (width 0.25) (layer "F.Cu") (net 8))
 (via (at 108.35 72.644) (size 0.8) (drill 0.4) (layers "F.Cu" "B.Cu") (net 8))
 (via (at 108.350614 78.232241) (size 0.8) (drill 0.4) (layers "F.Cu" "B.Cu") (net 8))
 (segment (start 108.35 78.231627) (end 108.350614 78.232241) (width 0.25) (layer "B.Cu") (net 8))
 (segment (start 108.35 72.644) (end 108.35 78.231627) (width 0.25) (layer "B.Cu") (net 8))
 (segment (start 118.675 79.65) (end 119.225 79.1) (width 0.25) (layer "F.Cu") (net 3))
 (segment (start 116.459999 73.17) (end 116.989999 73.7) (width 0.25) (layer "F.Cu") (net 3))
 (segment (start 115.95 73.17) (end 116.459999 73.17) (width 0.25) (layer "F.Cu") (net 3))
 (segment (start 119.225 79.1) (end 119.225 74.825) (width 0.25) (layer "F.Cu") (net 3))
 (segment (start 116.989999 73.7) (end 118.1 73.7) (width 0.25) (layer "F.Cu") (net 3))
 (segment (start 119.225 74.825) (end 118.1 73.7) (width 0.25) (layer "F.Cu") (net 3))
 (segment (start 115.95 73.17) (end 117.0675 73.17) (width 0.25) (layer "F.Cu") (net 3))
 (segment (start 117.0675 73.17) (end 118.6375 71.6) (width 0.25) (layer "F.Cu") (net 3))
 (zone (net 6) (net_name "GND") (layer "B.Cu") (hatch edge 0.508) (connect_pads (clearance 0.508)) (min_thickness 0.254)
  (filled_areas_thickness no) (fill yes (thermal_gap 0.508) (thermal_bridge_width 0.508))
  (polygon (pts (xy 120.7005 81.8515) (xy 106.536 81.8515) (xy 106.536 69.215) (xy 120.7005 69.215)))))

